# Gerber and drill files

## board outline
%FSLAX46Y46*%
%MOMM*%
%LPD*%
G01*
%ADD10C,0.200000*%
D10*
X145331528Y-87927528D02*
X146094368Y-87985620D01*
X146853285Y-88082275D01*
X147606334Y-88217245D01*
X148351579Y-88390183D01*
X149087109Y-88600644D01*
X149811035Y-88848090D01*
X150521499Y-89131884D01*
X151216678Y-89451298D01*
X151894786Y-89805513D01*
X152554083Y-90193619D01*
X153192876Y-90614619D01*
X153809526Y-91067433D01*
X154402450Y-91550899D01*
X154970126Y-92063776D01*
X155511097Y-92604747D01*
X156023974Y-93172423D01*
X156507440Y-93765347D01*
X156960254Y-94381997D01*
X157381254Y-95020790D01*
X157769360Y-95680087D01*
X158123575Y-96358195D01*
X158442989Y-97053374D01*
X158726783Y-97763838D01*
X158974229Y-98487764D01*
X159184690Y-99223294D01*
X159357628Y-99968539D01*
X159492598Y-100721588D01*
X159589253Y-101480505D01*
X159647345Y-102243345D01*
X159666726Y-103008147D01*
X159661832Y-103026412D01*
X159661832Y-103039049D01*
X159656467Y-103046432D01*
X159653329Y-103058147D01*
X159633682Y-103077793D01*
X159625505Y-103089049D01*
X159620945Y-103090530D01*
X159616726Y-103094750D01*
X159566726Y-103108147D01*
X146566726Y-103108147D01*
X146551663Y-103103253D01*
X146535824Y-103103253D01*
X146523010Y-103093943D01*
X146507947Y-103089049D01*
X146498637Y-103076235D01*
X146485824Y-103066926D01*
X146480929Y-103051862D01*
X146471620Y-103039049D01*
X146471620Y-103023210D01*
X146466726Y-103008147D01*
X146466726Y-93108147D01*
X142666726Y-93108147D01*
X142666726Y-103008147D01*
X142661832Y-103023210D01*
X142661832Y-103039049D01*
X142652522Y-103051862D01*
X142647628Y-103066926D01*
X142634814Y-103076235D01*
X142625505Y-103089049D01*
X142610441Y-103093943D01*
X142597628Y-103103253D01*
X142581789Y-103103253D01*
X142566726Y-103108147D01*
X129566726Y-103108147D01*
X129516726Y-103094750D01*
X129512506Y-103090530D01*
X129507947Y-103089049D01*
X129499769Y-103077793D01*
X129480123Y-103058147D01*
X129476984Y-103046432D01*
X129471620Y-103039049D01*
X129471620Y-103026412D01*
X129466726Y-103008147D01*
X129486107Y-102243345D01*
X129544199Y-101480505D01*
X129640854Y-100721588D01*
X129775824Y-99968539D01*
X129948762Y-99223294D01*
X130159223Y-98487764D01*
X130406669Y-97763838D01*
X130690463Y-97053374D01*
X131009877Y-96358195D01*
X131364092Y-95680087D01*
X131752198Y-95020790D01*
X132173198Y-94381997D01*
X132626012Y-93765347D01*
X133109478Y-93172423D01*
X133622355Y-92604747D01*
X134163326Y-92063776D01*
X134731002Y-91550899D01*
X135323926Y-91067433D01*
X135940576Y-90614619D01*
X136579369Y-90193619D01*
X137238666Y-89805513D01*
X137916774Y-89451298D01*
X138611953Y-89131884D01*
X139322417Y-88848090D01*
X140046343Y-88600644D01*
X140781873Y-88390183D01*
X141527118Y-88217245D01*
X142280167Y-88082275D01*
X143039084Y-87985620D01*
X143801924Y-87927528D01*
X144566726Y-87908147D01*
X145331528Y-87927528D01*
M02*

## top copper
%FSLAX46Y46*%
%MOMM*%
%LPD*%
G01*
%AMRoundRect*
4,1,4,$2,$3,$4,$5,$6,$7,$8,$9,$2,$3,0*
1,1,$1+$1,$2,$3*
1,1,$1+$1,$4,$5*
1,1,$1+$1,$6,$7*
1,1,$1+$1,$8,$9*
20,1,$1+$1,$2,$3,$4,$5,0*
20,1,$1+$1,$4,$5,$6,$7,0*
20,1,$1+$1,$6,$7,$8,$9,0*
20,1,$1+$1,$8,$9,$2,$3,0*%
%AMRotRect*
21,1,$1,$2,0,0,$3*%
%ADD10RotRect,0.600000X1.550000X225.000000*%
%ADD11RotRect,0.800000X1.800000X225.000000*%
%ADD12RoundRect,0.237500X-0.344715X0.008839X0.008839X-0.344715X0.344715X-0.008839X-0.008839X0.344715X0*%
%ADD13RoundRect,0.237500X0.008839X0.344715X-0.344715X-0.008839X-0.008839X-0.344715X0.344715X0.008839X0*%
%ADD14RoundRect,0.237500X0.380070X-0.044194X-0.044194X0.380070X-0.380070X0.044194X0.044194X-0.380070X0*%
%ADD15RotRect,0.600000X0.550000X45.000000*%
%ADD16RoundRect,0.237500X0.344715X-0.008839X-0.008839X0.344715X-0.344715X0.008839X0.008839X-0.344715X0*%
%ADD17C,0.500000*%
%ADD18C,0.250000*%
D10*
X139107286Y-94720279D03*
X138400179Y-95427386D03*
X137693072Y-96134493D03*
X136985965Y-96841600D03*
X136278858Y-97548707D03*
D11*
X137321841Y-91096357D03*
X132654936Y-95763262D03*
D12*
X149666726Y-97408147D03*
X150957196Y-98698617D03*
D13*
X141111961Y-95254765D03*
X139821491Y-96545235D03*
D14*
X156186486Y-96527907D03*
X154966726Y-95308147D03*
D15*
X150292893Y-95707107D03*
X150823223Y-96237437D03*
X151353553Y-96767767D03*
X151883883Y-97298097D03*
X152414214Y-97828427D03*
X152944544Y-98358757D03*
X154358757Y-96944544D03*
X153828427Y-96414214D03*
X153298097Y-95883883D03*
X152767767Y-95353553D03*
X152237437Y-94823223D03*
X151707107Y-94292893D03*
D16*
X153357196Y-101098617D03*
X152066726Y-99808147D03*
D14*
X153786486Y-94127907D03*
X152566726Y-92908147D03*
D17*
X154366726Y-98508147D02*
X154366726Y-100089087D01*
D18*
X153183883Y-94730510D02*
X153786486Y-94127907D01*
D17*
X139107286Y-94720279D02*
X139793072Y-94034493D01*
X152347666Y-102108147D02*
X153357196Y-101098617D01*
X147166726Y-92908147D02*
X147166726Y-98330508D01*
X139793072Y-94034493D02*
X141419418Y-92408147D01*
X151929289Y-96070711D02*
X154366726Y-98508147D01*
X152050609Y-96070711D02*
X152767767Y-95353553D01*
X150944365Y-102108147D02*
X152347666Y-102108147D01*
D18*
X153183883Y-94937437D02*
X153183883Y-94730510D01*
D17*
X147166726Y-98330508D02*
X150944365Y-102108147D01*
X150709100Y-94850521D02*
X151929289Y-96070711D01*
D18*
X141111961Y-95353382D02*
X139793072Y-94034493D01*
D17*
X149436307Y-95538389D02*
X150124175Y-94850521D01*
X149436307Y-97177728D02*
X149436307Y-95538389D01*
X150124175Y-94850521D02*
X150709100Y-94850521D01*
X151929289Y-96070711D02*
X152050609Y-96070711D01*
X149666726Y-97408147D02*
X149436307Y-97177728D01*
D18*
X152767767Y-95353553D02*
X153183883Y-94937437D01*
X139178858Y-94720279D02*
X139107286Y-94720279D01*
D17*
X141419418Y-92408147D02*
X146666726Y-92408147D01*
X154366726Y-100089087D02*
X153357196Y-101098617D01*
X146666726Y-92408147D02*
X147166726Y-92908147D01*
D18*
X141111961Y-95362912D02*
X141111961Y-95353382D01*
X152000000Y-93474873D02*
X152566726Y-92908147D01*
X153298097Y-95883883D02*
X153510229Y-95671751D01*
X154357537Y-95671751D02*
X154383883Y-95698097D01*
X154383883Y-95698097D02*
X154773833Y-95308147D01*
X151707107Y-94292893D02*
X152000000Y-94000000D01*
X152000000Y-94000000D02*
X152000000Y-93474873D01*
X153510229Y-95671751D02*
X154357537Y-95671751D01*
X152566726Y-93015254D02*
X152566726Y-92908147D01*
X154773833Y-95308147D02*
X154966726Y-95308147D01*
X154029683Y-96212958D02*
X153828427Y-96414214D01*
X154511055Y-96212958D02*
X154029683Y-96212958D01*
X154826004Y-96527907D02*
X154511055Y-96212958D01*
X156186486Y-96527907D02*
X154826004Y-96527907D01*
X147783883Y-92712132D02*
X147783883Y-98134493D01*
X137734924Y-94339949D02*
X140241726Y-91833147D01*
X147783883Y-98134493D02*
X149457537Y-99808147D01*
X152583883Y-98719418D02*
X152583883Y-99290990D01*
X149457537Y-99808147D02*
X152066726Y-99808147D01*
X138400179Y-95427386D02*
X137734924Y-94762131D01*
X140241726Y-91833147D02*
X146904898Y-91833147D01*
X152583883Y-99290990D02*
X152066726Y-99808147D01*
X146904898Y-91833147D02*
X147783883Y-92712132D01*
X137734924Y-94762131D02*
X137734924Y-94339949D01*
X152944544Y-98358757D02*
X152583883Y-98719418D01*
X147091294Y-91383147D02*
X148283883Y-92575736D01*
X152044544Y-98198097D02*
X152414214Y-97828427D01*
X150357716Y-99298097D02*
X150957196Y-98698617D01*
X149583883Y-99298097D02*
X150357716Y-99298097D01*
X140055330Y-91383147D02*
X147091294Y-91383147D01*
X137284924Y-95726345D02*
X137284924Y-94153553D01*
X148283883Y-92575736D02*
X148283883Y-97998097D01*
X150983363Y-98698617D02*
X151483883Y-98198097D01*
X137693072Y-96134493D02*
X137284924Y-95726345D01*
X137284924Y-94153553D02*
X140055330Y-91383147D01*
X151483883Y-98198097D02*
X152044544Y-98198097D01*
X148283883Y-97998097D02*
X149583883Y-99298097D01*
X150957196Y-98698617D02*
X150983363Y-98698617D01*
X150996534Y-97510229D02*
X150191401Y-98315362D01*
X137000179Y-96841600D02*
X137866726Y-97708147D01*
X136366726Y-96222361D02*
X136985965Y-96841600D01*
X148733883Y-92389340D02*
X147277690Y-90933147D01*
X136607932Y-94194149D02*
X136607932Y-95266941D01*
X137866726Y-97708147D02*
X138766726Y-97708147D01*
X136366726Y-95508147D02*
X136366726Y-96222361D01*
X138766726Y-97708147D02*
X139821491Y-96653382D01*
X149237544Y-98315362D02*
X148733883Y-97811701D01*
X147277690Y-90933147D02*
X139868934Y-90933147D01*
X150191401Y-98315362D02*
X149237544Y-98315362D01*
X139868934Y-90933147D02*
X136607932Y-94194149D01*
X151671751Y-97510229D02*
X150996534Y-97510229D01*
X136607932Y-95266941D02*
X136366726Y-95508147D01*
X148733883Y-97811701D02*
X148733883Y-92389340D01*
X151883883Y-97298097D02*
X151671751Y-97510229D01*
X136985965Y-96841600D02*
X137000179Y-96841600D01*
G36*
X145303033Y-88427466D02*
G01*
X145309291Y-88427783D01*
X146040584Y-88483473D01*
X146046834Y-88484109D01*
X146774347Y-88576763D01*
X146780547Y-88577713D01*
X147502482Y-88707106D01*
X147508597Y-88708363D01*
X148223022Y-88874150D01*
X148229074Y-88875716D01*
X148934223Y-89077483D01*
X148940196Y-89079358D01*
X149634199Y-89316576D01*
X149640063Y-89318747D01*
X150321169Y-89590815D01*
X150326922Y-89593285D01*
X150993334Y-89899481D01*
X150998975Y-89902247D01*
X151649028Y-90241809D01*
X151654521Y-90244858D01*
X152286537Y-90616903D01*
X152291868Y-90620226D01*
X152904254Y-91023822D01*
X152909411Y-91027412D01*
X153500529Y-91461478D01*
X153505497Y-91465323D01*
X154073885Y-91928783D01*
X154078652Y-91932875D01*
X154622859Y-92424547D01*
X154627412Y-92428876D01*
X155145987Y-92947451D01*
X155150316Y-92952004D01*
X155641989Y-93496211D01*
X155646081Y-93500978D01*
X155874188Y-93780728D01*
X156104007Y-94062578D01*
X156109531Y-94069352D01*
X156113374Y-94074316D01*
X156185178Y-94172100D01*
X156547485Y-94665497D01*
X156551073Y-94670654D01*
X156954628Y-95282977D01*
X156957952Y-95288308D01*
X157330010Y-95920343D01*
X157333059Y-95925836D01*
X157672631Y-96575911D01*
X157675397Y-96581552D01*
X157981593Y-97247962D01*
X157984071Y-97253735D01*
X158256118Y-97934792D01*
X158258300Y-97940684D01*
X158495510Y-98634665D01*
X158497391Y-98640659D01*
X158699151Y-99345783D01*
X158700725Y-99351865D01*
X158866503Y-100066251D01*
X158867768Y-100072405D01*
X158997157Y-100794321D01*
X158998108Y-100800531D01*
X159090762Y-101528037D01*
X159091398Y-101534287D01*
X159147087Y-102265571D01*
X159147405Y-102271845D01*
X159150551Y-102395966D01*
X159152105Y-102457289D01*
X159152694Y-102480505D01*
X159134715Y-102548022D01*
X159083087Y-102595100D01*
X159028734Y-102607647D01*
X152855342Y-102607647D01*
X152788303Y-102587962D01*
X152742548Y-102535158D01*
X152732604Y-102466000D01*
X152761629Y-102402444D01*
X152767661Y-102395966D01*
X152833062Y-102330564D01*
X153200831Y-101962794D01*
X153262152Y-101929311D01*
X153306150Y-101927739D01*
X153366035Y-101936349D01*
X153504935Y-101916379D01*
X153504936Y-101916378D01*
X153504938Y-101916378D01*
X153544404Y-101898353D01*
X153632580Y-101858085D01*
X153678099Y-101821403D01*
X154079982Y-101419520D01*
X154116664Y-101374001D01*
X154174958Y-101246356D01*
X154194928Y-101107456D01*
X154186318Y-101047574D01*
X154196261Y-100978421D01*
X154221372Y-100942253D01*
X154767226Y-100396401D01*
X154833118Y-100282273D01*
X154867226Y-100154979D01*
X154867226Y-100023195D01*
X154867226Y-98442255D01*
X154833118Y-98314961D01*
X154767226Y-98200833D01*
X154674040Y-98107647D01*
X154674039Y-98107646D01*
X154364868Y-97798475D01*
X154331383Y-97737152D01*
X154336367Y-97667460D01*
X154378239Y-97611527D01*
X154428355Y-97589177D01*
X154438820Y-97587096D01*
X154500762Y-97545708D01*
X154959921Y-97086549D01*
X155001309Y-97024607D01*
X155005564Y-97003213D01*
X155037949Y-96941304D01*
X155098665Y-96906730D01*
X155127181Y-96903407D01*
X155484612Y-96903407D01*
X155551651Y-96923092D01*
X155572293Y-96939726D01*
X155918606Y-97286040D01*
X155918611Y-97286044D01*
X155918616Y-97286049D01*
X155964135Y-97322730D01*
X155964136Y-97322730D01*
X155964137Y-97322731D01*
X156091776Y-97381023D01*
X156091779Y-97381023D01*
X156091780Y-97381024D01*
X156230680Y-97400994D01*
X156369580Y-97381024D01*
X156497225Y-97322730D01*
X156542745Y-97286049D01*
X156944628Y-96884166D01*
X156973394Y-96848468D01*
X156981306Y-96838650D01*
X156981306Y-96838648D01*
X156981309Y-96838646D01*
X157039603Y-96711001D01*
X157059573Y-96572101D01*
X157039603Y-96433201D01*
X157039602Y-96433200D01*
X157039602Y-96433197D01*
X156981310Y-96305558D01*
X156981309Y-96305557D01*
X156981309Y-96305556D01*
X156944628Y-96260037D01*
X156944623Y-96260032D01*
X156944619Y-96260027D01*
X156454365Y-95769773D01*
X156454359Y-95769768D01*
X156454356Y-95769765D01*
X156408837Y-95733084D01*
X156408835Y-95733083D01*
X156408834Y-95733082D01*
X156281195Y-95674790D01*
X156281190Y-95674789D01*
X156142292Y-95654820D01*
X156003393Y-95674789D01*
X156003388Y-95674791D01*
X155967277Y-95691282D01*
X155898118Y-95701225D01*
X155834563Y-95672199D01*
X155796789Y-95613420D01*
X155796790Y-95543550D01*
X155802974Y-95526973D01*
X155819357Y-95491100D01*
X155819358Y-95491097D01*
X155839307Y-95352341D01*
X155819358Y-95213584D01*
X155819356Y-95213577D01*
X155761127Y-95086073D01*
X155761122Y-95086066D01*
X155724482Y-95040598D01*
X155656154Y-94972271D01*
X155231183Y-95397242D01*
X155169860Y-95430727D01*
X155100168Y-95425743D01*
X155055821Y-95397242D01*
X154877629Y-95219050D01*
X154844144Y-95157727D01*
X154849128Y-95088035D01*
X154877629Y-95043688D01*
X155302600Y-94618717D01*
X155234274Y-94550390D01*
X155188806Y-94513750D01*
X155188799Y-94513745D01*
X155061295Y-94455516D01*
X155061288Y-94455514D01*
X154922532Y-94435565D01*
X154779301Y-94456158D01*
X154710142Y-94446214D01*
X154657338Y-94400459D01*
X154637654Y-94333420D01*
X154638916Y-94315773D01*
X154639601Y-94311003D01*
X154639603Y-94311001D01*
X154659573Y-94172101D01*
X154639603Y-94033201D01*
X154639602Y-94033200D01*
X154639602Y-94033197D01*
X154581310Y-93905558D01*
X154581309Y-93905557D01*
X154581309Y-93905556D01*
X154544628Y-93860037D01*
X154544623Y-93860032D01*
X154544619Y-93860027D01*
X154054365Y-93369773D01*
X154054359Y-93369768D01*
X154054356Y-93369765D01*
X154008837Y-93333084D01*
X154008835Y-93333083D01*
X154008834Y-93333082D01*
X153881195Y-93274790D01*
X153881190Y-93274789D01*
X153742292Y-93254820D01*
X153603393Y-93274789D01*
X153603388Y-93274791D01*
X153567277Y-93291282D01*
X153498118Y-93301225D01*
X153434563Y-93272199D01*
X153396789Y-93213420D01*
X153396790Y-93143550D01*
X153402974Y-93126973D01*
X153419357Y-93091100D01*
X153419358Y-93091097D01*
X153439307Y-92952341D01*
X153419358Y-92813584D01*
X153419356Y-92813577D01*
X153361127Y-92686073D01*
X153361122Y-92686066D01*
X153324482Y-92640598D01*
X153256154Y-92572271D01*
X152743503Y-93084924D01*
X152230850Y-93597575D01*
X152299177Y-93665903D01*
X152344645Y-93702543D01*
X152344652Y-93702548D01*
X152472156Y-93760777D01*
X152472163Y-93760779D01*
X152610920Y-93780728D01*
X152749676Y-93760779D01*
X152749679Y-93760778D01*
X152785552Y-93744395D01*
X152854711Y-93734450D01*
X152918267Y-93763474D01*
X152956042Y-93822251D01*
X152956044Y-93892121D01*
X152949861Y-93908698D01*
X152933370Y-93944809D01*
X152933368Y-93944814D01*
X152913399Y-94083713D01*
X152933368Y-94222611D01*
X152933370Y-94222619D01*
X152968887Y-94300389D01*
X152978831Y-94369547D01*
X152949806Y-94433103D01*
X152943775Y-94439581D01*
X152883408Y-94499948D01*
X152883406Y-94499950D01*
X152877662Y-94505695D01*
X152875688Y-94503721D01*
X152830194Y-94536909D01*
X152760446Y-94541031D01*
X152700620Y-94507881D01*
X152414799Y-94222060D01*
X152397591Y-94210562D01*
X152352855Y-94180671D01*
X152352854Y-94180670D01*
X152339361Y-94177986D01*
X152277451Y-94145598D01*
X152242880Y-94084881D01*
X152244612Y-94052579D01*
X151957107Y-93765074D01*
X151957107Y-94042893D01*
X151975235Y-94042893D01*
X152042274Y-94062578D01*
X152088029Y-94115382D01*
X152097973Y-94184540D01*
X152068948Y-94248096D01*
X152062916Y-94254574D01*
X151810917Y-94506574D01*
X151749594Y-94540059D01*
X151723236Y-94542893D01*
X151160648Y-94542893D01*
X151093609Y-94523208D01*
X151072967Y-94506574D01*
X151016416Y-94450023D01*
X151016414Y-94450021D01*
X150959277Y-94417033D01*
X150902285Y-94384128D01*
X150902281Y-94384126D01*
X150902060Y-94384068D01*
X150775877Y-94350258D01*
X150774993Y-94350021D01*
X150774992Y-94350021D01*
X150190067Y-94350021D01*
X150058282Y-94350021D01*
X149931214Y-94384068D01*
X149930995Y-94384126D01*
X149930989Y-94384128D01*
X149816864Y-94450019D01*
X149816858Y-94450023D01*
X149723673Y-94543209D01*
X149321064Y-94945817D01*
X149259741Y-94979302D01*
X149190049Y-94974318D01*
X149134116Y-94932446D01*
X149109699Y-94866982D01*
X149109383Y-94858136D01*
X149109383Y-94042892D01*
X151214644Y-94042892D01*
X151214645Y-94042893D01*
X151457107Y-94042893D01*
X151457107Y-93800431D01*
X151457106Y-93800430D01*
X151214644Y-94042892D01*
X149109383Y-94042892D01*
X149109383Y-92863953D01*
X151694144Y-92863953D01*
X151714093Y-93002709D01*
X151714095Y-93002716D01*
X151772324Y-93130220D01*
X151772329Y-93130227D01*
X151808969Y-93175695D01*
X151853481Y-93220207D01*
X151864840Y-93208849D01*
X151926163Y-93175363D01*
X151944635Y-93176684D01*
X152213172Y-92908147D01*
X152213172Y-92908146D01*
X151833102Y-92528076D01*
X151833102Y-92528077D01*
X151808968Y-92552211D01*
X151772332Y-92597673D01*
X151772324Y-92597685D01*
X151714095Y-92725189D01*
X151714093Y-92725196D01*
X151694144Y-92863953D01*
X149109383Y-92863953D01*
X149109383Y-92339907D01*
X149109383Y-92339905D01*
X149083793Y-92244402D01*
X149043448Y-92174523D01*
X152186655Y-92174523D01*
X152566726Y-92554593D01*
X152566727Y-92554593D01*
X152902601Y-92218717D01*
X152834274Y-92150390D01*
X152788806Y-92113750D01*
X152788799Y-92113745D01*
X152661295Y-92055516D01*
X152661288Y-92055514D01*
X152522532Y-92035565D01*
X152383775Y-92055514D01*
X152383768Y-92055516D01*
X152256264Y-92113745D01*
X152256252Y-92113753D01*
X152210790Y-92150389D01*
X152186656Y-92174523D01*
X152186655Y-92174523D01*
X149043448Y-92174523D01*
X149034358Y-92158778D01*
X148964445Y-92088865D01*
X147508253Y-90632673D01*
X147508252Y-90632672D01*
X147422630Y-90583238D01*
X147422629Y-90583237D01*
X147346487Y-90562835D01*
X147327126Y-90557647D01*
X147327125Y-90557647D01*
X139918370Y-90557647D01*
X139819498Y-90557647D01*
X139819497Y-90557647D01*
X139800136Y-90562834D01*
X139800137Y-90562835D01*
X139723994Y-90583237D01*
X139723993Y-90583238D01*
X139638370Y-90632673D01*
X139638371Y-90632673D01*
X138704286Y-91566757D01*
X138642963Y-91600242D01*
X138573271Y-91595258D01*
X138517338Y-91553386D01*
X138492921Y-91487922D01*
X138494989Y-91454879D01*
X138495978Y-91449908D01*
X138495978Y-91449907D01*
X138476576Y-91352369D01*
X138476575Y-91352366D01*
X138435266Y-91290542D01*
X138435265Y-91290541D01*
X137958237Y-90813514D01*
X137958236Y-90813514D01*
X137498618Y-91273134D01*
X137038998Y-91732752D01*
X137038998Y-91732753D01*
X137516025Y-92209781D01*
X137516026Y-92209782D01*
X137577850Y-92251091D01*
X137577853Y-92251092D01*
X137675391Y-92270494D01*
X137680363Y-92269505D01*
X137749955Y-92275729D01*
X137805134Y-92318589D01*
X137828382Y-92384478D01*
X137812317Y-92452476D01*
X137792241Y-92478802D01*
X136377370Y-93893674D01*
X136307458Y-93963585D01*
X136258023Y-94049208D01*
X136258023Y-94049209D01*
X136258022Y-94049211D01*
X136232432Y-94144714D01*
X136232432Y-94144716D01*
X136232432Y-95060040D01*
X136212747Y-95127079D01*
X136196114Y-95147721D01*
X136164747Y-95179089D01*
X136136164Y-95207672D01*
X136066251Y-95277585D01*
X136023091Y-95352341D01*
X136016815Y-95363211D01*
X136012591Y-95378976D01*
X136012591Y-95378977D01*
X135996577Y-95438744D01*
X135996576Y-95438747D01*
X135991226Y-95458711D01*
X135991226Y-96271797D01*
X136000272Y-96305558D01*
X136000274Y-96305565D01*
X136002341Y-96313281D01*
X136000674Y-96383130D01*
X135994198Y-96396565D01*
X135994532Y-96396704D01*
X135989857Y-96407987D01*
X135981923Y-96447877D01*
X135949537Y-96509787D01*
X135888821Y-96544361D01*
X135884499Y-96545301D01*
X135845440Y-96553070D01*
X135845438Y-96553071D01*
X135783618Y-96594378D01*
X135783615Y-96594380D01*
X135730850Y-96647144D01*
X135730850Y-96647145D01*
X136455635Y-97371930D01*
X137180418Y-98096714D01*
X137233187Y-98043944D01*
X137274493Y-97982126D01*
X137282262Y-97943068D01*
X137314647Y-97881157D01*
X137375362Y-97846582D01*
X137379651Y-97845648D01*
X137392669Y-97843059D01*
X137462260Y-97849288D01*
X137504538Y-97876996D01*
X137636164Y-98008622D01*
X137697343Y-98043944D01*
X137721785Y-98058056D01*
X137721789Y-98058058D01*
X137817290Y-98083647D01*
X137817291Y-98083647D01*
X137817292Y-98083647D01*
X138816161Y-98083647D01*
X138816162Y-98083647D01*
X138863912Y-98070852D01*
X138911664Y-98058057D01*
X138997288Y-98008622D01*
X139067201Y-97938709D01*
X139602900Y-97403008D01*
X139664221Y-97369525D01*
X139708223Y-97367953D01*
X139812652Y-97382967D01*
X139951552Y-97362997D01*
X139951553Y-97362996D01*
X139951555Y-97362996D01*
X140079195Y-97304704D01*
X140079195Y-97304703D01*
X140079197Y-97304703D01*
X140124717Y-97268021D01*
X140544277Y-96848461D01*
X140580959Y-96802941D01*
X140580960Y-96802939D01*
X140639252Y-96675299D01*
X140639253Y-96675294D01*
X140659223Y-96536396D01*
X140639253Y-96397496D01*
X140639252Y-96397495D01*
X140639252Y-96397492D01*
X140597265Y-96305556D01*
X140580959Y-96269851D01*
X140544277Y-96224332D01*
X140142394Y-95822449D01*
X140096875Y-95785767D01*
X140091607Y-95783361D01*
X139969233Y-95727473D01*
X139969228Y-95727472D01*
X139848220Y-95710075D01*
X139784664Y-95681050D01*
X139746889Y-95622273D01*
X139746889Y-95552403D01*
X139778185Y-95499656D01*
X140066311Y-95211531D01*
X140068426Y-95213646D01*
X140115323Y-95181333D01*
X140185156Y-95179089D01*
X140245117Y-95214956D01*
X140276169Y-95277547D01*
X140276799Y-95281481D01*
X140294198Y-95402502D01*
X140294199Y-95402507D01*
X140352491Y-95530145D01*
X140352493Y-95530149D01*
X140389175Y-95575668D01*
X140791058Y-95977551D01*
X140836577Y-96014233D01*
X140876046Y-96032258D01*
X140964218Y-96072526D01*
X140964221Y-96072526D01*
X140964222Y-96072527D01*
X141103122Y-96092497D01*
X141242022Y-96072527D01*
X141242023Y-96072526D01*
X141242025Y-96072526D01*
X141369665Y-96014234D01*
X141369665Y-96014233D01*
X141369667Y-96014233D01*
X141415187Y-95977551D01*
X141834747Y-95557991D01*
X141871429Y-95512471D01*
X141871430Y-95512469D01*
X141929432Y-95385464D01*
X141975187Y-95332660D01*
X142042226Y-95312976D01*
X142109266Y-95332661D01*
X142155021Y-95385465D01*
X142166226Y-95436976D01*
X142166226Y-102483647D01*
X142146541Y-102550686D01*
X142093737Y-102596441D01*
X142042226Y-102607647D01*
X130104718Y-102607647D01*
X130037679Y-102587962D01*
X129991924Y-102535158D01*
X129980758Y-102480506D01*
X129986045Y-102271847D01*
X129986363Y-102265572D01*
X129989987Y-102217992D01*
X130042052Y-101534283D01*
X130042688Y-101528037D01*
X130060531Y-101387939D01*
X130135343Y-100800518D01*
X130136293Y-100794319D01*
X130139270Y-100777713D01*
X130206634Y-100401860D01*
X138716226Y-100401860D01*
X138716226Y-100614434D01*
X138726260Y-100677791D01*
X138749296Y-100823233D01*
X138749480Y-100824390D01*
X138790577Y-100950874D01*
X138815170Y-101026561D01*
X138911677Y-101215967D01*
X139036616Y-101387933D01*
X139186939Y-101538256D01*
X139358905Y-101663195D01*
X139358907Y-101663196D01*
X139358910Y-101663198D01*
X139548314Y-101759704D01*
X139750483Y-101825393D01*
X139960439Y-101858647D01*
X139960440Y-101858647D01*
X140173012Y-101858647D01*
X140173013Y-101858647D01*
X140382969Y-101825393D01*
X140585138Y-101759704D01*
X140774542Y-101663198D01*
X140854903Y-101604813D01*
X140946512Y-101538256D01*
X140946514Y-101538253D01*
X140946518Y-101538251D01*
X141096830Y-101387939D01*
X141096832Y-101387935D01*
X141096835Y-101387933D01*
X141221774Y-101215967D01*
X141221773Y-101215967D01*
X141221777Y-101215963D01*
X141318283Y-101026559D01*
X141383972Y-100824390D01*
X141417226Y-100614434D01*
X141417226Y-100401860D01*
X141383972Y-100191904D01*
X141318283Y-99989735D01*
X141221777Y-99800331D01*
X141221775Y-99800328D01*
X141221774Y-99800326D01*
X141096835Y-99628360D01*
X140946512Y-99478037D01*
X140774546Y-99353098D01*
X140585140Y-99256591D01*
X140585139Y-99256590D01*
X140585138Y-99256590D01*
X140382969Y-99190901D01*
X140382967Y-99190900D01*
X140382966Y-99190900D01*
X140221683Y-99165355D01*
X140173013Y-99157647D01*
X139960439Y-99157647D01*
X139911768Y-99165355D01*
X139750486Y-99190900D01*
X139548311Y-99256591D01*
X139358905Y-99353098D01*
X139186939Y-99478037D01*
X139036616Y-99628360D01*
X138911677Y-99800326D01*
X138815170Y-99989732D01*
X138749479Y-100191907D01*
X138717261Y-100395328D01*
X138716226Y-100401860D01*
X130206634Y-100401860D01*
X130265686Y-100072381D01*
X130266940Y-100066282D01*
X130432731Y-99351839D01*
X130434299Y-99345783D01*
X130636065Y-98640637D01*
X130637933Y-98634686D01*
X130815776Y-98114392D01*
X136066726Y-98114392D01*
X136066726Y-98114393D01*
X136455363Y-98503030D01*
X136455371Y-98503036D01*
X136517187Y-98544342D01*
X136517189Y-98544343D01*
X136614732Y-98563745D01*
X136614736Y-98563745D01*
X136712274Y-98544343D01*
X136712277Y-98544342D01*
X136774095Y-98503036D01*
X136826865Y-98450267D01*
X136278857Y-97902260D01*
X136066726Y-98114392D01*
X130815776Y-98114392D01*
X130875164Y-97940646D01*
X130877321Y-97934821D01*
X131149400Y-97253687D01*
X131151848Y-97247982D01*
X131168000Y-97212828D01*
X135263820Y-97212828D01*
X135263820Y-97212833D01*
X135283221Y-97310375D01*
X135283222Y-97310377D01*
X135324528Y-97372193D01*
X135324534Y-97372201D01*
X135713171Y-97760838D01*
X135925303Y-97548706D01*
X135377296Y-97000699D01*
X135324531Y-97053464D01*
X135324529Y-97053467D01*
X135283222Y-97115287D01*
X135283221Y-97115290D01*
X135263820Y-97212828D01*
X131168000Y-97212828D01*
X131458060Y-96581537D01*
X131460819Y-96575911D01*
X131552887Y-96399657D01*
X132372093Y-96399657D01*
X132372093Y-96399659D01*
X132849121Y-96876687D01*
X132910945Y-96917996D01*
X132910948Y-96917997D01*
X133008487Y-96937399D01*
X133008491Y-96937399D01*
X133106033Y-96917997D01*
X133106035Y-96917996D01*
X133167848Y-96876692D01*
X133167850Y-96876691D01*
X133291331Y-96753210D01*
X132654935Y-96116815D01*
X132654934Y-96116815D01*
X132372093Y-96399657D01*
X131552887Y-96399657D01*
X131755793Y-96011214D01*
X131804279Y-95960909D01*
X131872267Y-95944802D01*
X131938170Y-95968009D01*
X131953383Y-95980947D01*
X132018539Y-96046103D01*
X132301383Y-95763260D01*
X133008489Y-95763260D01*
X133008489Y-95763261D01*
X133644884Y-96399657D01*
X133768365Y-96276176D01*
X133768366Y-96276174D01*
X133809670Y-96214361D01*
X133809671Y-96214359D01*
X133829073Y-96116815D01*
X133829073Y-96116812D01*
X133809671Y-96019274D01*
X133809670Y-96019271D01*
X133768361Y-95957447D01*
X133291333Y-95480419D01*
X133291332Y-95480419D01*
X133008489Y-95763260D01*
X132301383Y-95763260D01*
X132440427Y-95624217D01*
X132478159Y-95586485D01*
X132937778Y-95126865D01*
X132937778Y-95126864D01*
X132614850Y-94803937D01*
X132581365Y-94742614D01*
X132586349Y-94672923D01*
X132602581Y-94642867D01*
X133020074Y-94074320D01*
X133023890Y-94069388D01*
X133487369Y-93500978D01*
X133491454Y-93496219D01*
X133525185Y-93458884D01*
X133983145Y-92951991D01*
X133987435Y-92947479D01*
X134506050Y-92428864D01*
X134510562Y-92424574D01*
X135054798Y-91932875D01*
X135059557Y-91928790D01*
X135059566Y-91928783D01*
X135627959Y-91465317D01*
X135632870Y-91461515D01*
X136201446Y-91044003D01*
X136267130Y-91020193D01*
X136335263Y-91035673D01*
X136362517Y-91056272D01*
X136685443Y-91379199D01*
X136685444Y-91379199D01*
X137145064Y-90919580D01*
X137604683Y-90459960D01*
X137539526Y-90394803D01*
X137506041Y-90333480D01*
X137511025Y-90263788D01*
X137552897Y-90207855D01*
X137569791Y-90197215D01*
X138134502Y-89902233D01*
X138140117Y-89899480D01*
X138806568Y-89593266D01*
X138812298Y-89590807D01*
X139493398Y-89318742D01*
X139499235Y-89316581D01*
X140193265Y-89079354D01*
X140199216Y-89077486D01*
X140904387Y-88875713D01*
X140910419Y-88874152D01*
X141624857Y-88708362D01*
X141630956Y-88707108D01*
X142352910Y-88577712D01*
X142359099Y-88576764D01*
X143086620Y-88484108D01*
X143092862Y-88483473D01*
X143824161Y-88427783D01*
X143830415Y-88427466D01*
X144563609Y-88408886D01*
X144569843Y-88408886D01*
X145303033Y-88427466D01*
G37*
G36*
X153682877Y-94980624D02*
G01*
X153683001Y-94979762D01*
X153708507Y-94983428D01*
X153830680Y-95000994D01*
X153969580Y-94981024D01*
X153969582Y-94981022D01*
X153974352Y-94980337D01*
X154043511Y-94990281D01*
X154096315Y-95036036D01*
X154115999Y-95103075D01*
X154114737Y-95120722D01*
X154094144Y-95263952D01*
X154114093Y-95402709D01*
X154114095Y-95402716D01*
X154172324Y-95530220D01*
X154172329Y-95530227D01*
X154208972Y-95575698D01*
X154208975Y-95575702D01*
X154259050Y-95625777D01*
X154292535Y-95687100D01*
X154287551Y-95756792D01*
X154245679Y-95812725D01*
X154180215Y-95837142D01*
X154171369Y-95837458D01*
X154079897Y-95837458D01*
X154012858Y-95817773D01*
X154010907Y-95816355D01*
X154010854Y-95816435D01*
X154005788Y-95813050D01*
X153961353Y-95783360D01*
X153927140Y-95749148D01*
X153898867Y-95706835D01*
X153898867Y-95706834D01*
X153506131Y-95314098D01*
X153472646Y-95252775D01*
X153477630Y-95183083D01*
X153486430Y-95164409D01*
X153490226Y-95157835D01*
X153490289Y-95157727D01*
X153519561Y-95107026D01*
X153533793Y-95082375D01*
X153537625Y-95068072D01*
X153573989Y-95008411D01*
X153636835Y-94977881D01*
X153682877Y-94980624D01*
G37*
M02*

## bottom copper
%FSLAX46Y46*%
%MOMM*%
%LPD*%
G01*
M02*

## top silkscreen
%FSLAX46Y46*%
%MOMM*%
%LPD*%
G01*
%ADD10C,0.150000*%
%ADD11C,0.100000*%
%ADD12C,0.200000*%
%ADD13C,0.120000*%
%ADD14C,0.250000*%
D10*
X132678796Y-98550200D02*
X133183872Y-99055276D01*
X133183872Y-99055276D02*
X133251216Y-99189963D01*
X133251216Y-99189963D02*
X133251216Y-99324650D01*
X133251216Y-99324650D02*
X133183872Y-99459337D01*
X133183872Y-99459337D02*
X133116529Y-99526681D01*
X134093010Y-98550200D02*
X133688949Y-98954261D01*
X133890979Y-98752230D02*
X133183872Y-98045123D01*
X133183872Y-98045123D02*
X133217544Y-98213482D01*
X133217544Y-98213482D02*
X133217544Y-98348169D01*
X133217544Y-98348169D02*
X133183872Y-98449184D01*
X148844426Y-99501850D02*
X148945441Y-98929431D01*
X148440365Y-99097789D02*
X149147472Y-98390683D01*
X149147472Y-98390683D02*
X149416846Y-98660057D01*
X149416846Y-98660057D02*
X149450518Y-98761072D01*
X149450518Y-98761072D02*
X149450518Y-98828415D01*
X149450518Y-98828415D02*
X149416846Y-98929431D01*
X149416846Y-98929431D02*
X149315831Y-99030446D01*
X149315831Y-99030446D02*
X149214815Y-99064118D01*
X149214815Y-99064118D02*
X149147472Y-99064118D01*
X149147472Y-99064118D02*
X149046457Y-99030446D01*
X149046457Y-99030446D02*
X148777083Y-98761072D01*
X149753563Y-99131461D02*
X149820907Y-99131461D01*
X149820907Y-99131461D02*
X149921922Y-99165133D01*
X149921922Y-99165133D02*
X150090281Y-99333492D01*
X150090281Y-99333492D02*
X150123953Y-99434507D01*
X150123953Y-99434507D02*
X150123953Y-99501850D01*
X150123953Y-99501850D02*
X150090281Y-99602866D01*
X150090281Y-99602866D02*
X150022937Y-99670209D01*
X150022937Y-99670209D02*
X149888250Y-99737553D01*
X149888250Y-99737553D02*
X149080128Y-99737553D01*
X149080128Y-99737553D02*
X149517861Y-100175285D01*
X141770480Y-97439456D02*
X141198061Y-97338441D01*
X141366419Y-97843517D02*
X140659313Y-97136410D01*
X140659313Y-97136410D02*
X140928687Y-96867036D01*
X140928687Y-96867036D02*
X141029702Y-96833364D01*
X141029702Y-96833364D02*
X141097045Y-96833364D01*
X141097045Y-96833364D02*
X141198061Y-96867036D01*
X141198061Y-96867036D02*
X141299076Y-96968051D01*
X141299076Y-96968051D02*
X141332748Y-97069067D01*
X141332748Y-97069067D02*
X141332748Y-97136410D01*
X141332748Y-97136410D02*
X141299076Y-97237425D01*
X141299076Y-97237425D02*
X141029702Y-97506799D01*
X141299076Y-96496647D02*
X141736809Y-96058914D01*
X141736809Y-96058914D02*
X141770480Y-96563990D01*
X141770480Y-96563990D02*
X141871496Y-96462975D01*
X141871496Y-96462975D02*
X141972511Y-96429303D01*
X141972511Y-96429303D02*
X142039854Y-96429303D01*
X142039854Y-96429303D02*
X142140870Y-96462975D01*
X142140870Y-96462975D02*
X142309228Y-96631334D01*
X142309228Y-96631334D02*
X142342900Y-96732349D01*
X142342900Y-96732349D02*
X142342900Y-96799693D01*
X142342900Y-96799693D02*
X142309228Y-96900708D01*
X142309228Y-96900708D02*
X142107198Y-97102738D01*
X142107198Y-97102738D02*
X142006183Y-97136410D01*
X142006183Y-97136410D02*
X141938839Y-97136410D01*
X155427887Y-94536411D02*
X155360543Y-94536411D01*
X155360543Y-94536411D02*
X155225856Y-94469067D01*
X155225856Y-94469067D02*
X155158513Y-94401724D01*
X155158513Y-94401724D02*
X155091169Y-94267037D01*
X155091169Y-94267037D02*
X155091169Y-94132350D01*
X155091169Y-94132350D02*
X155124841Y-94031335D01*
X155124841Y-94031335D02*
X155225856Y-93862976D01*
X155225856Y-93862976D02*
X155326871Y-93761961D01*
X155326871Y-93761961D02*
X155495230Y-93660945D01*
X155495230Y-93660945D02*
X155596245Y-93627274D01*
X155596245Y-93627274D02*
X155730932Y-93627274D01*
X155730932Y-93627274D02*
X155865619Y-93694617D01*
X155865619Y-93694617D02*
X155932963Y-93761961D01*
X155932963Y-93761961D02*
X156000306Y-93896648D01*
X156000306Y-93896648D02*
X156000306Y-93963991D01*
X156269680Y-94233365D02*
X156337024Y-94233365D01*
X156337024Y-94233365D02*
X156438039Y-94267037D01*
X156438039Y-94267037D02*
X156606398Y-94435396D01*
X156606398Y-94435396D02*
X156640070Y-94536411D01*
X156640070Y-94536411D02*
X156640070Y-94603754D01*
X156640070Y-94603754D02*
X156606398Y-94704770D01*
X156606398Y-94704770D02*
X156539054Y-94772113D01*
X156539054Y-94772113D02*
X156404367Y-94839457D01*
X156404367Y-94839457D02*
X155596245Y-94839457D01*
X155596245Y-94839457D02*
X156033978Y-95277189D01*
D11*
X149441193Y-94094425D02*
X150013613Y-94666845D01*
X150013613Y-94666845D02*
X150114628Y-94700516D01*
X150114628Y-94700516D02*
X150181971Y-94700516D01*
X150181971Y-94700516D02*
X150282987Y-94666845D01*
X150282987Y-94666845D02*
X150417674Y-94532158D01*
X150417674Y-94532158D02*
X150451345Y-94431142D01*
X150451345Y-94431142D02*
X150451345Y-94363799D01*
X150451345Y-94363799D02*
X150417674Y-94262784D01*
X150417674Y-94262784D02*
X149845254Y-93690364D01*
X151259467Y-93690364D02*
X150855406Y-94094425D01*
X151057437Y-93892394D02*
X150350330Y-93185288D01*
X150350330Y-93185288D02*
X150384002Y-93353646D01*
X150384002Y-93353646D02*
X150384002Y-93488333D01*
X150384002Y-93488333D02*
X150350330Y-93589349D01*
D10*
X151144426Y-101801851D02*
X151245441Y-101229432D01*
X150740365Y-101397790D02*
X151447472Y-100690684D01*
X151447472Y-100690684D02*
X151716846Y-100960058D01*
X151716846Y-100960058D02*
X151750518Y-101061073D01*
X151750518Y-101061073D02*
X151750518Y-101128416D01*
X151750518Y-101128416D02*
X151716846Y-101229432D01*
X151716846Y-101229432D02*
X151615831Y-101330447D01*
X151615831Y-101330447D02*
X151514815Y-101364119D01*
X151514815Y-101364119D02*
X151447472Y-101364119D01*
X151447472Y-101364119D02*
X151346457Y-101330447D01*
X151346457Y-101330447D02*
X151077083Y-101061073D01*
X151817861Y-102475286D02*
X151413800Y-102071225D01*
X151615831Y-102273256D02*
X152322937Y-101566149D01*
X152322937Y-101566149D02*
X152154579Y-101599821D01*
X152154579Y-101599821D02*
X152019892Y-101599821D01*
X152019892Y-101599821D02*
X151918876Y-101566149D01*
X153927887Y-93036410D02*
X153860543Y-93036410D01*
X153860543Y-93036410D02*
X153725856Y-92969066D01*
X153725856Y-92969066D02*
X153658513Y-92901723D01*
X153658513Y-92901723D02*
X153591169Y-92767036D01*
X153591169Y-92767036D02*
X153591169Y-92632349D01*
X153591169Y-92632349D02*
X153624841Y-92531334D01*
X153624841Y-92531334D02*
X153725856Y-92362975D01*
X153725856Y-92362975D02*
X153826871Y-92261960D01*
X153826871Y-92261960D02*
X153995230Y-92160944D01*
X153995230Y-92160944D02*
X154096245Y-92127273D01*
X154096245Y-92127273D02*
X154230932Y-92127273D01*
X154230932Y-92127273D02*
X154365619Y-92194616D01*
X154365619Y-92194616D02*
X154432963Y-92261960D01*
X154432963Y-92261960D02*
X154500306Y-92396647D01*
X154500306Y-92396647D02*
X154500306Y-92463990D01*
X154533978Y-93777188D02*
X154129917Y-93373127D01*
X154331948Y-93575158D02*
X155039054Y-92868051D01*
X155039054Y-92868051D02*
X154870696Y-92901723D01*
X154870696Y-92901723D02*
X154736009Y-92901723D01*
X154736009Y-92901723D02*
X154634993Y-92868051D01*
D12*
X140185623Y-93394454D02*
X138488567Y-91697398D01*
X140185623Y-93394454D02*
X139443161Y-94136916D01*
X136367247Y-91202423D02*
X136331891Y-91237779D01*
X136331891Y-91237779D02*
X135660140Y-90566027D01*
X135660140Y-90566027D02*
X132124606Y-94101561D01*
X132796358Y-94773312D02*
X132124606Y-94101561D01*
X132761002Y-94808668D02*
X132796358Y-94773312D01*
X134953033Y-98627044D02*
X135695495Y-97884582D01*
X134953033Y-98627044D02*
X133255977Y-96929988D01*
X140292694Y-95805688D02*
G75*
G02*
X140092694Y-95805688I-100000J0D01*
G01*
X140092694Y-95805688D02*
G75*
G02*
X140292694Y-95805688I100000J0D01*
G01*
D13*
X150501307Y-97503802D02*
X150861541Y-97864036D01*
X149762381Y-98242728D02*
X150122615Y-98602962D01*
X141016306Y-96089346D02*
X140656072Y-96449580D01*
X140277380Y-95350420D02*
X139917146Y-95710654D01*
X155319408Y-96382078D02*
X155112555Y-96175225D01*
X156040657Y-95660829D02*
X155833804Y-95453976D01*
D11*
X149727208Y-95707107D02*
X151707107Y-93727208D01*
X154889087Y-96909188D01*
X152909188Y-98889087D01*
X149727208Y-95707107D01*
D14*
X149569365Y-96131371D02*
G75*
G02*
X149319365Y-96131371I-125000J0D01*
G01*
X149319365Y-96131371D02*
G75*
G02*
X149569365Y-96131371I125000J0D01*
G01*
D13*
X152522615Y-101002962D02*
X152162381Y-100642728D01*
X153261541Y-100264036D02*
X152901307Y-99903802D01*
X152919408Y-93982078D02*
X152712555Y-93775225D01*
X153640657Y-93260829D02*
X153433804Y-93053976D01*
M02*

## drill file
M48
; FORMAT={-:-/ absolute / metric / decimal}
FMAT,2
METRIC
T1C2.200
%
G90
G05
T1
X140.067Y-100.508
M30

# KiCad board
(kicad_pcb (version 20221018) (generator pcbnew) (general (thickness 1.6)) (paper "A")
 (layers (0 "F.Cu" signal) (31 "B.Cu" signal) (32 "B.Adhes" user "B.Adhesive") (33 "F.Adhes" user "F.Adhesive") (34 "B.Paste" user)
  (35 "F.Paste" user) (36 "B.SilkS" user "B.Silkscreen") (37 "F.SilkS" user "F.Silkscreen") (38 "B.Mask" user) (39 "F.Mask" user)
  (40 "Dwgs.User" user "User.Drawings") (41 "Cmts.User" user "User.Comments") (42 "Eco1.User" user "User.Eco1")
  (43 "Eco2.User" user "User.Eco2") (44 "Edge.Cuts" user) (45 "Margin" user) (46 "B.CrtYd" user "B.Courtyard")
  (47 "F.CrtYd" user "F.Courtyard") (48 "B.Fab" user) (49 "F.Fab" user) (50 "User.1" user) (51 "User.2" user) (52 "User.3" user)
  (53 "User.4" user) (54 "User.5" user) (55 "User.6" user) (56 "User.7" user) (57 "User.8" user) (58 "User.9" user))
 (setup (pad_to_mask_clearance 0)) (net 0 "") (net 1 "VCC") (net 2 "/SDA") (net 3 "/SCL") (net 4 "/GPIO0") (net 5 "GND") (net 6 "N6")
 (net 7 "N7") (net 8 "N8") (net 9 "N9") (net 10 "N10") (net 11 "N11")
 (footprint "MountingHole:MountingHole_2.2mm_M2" (layer "F.Cu") (at 140.066726 100.508147)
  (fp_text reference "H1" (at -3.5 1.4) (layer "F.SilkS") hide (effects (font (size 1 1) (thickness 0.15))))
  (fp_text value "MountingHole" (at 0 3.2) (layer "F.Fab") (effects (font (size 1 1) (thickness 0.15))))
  (pad "" np_thru_hole circle (at 0 0) (size 2.2 2.2) (drill 2.2) (layers "*.Cu" "*.Mask")))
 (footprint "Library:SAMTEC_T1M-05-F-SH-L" (layer "F.Cu") (at 137.693072 96.134493 -135)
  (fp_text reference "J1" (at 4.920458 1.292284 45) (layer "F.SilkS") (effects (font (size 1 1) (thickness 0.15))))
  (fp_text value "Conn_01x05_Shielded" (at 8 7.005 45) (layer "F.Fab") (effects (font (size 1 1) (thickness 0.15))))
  (fp_line (start -3.7 0.175) (end -3.7 2.575) (stroke (width 0.2) (type solid)) (layer "F.SilkS"))
  (fp_line (start -3.7 0.175) (end -2.65 0.175) (stroke (width 0.2) (type solid)) (layer "F.SilkS"))
  (fp_line (start -2.55 4.425) (end -2.5 4.425) (stroke (width 0.2) (type solid)) (layer "F.SilkS"))
  (fp_line (start -2.5 4.425) (end -2.5 5.375) (stroke (width 0.2) (type solid)) (layer "F.SilkS"))
  (fp_line (start -2.5 5.375) (end 2.5 5.375) (stroke (width 0.2) (type solid)) (layer "F.SilkS"))
  (fp_line (start 2.5 4.425) (end 2.5 5.375) (stroke (width 0.2) (type solid)) (layer "F.SilkS"))
  (fp_line (start 2.55 4.425) (end 2.5 4.425) (stroke (width 0.2) (type solid)) (layer "F.SilkS"))
  (fp_line (start 3.7 0.175) (end 2.65 0.175) (stroke (width 0.2) (type solid)) (layer "F.SilkS"))
  (fp_line (start 3.7 0.175) (end 3.7 2.575) (stroke (width 0.2) (type solid)) (layer "F.SilkS"))
  (fp_circle (center -2 -1.535) (end -1.9 -1.535) (stroke (width 0.2) (type solid)) (fill none) (layer "F.SilkS"))
  (pad "1" smd rect (at -2 0 225) (size 0.6 1.55) (layers "F.Cu" "F.Paste" "F.Mask") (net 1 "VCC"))
  (pad "2" smd rect (at -1 0 225) (size 0.6 1.55) (layers "F.Cu" "F.Paste" "F.Mask") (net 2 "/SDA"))
  (pad "3" smd rect (at 0 0 225) (size 0.6 1.55) (layers "F.Cu" "F.Paste" "F.Mask") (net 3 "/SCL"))
  (pad "4" smd rect (at 1 0 225) (size 0.6 1.55) (layers "F.Cu" "F.Paste" "F.Mask") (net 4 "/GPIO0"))
  (pad "5" smd rect (at 2 0 225) (size 0.6 1.55) (layers "F.Cu" "F.Paste" "F.Mask") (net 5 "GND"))
  (pad "SH1" smd rect (at -3.3 3.825 225) (size 0.8 1.8) (layers "F.Cu" "F.Paste" "F.Mask") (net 5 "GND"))
  (pad "SH2" smd rect (at 3.3 3.825 225) (size 0.8 1.8) (layers "F.Cu" "F.Paste" "F.Mask") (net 5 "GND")))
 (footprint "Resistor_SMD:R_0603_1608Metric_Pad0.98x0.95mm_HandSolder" (layer "F.Cu") (at 150.311961 98.053382 -45)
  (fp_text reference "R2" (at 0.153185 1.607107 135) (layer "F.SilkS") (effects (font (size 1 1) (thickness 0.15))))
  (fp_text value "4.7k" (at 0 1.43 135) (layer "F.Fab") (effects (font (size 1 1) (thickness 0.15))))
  (fp_line (start -0.254724 -0.5225) (end 0.254724 -0.5225) (stroke (width 0.12) (type solid)) (layer "F.SilkS"))
  (fp_line (start -0.254724 0.5225) (end 0.254724 0.5225) (stroke (width 0.12) (type solid)) (layer "F.SilkS"))
  (pad "1" smd roundrect (at -0.9125 0 315) (size 0.975 0.95) (layers "F.Cu" "F.Paste" "F.Mask") (roundrect_rratio 0.25) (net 1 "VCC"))
  (pad "2" smd roundrect (at 0.9125 0 315) (size 0.975 0.95) (layers "F.Cu" "F.Paste" "F.Mask") (roundrect_rratio 0.25) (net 3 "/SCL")))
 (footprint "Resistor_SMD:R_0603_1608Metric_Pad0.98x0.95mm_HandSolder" (layer "F.Cu") (at 140.466726 95.9 -135)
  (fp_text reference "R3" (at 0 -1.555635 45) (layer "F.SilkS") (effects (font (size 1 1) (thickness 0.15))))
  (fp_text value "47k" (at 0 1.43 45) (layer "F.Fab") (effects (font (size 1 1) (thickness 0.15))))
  (fp_line (start -0.254724 -0.5225) (end 0.254724 -0.5225) (stroke (width 0.12) (type solid)) (layer "F.SilkS"))
  (fp_line (start -0.254724 0.5225) (end 0.254724 0.5225) (stroke (width 0.12) (type solid)) (layer "F.SilkS"))
  (pad "1" smd roundrect (at -0.9125 0 225) (size 0.975 0.95) (layers "F.Cu" "F.Paste" "F.Mask") (roundrect_rratio 0.25) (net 1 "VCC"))
  (pad "2" smd roundrect (at 0.9125 0 225) (size 0.975 0.95) (layers "F.Cu" "F.Paste" "F.Mask") (roundrect_rratio 0.25) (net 4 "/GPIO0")))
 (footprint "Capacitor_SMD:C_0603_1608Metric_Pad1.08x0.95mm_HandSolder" (layer "F.Cu") (at 155.576606 95.918027 135)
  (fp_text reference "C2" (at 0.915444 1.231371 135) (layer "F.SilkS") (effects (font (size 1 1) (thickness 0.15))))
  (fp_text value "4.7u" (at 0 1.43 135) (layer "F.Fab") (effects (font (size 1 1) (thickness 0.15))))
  (fp_line (start -0.146267 -0.51) (end 0.146267 -0.51) (stroke (width 0.12) (type solid)) (layer "F.SilkS"))
  (fp_line (start -0.146267 0.51) (end 0.146267 0.51) (stroke (width 0.12) (type solid)) (layer "F.SilkS"))
  (pad "1" smd roundrect (at -0.8625 0 135) (size 1.075 0.95) (layers "F.Cu" "F.Paste" "F.Mask") (roundrect_rratio 0.25) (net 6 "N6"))
  (pad "2" smd roundrect (at 0.8625 0 135) (size 1.075 0.95) (layers "F.Cu" "F.Paste" "F.Mask") (roundrect_rratio 0.25) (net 5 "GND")))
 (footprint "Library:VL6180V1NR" (layer "F.Cu") (at 151 95 45)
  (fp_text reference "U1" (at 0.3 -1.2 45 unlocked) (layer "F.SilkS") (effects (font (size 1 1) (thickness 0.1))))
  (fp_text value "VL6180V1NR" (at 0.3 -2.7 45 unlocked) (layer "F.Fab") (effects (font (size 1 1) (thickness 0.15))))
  (fp_rect (start -1.4 -0.4) (end 1.4 4.1) (stroke (width 0.1) (type default)) (fill none) (layer "F.SilkS"))
  (fp_circle (center -1.9 -0.3) (end -1.7 -0.3) (stroke (width 0.1) (type solid)) (fill solid) (layer "F.SilkS"))
  (pad "1" smd rect (at -1 0 45) (size 0.6 0.55) (layers "F.Cu" "F.Paste" "F.Mask") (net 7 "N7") (thermal_bridge_angle 45))
  (pad "2" smd rect (at -1 0.75 45) (size 0.6 0.55) (layers "F.Cu" "F.Paste" "F.Mask") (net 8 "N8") (thermal_bridge_angle 45))
  (pad "3" smd rect (at -1 1.5 45) (size 0.6 0.55) (layers "F.Cu" "F.Paste" "F.Mask") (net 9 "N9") (thermal_bridge_angle 45))
  (pad "4" smd rect (at -1 2.25 45) (size 0.6 0.55) (layers "F.Cu" "F.Paste" "F.Mask") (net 4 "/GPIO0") (thermal_bridge_angle 45))
  (pad "5" smd rect (at -1 3 45) (size 0.6 0.55) (layers "F.Cu" "F.Paste" "F.Mask") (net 3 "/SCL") (thermal_bridge_angle 45))
  (pad "6" smd rect (at -1 3.75 45) (size 0.6 0.55) (layers "F.Cu" "F.Paste" "F.Mask") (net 2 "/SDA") (thermal_bridge_angle 45))
  (pad "7" smd rect (at 1 3.75 45) (size 0.6 0.55) (layers "F.Cu" "F.Paste" "F.Mask") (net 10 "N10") (thermal_bridge_angle 45))
  (pad "8" smd rect (at 1 3 45) (size 0.6 0.55) (layers "F.Cu" "F.Paste" "F.Mask") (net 6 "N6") (thermal_bridge_angle 45))
  (pad "9" smd rect (at 1 2.25 45) (size 0.6 0.55) (layers "F.Cu" "F.Paste" "F.Mask") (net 5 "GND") (thermal_bridge_angle 45))
  (pad "10" smd rect (at 1 1.5 45) (size 0.6 0.55) (layers "F.Cu" "F.Paste" "F.Mask") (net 1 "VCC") (thermal_bridge_angle 45))
  (pad "11" smd rect (at 1 0.75 45) (size 0.6 0.55) (layers "F.Cu" "F.Paste" "F.Mask") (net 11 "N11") (thermal_bridge_angle 45))
  (pad "12" smd rect (at 1 0 45) (size 0.6 0.55) (layers "F.Cu" "F.Paste" "F.Mask") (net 5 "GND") (thermal_bridge_angle 45)))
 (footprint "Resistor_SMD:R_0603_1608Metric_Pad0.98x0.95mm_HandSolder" (layer "F.Cu") (at 152.711961 100.453382 135)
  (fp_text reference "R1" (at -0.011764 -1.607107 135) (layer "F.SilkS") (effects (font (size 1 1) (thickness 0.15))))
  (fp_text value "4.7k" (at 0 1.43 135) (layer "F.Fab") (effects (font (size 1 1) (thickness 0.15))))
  (fp_line (start -0.254724 -0.5225) (end 0.254724 -0.5225) (stroke (width 0.12) (type solid)) (layer "F.SilkS"))
  (fp_line (start -0.254724 0.5225) (end 0.254724 0.5225) (stroke (width 0.12) (type solid)) (layer "F.SilkS"))
  (pad "1" smd roundrect (at -0.9125 0 135) (size 0.975 0.95) (layers "F.Cu" "F.Paste" "F.Mask") (roundrect_rratio 0.25) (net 1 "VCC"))
  (pad "2" smd roundrect (at 0.9125 0 135) (size 0.975 0.95) (layers "F.Cu" "F.Paste" "F.Mask") (roundrect_rratio 0.25) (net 2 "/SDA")))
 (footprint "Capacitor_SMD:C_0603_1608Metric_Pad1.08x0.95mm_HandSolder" (layer "F.Cu") (at 153.176606 93.518027 135)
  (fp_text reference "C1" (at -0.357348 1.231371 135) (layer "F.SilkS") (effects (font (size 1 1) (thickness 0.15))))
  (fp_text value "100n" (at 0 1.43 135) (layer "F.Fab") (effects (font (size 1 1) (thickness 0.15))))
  (fp_line (start -0.146267 -0.51) (end 0.146267 -0.51) (stroke (width 0.12) (type solid)) (layer "F.SilkS"))
  (fp_line (start -0.146267 0.51) (end 0.146267 0.51) (stroke (width 0.12) (type solid)) (layer "F.SilkS"))
  (pad "1" smd roundrect (at -0.8625 0 135) (size 1.075 0.95) (layers "F.Cu" "F.Paste" "F.Mask") (roundrect_rratio 0.25) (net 1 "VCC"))
  (pad "2" smd roundrect (at 0.8625 0 135) (size 1.075 0.95) (layers "F.Cu" "F.Paste" "F.Mask") (roundrect_rratio 0.25) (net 5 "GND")))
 (gr_poly
  (pts (xy 145.331528 87.927528) (xy 146.094368 87.98562) (xy 146.853285 88.082275) (xy 147.606334 88.217245) (xy 148.351579 88.390183)
   (xy 149.087109 88.600644) (xy 149.811035 88.84809) (xy 150.521499 89.131884) (xy 151.216678 89.451298) (xy 151.894786 89.805513)
   (xy 152.554083 90.193619) (xy 153.192876 90.614619) (xy 153.809526 91.067433) (xy 154.40245 91.550899) (xy 154.970126 92.063776)
   (xy 155.511097 92.604747) (xy 156.023974 93.172423) (xy 156.50744 93.765347) (xy 156.960254 94.381997) (xy 157.381254 95.02079)
   (xy 157.76936 95.680087) (xy 158.123575 96.358195) (xy 158.442989 97.053374) (xy 158.726783 97.763838) (xy 158.974229 98.487764)
   (xy 159.18469 99.223294) (xy 159.357628 99.968539) (xy 159.492598 100.721588) (xy 159.589253 101.480505) (xy 159.647345 102.243345)
   (xy 159.666726 103.008147) (xy 159.661832 103.026412) (xy 159.661832 103.039049) (xy 159.656467 103.046432) (xy 159.653329 103.058147)
   (xy 159.633682 103.077793) (xy 159.625505 103.089049) (xy 159.620945 103.09053) (xy 159.616726 103.09475) (xy 159.566726 103.108147)
   (xy 146.566726 103.108147) (xy 146.551663 103.103253) (xy 146.535824 103.103253) (xy 146.52301 103.093943) (xy 146.507947 103.089049)
   (xy 146.498637 103.076235) (xy 146.485824 103.066926) (xy 146.480929 103.051862) (xy 146.47162 103.039049) (xy 146.47162 103.02321)
   (xy 146.466726 103.008147) (xy 146.466726 93.108147) (xy 142.666726 93.108147) (xy 142.666726 103.008147) (xy 142.661832 103.02321)
   (xy 142.661832 103.039049) (xy 142.652522 103.051862) (xy 142.647628 103.066926) (xy 142.634814 103.076235) (xy 142.625505 103.089049)
   (xy 142.610441 103.093943) (xy 142.597628 103.103253) (xy 142.581789 103.103253) (xy 142.566726 103.108147) (xy 129.566726 103.108147)
   (xy 129.516726 103.09475) (xy 129.512506 103.09053) (xy 129.507947 103.089049) (xy 129.499769 103.077793) (xy 129.480123 103.058147)
   (xy 129.476984 103.046432) (xy 129.47162 103.039049) (xy 129.47162 103.026412) (xy 129.466726 103.008147) (xy 129.486107 102.243345)
   (xy 129.544199 101.480505) (xy 129.640854 100.721588) (xy 129.775824 99.968539) (xy 129.948762 99.223294) (xy 130.159223 98.487764)
   (xy 130.406669 97.763838) (xy 130.690463 97.053374) (xy 131.009877 96.358195) (xy 131.364092 95.680087) (xy 131.752198 95.02079)
   (xy 132.173198 94.381997) (xy 132.626012 93.765347) (xy 133.109478 93.172423) (xy 133.622355 92.604747) (xy 134.163326 92.063776)
   (xy 134.731002 91.550899) (xy 135.323926 91.067433) (xy 135.940576 90.614619) (xy 136.579369 90.193619) (xy 137.238666 89.805513)
   (xy 137.916774 89.451298) (xy 138.611953 89.131884) (xy 139.322417 88.84809) (xy 140.046343 88.600644) (xy 140.781873 88.390183)
   (xy 141.527118 88.217245) (xy 142.280167 88.082275) (xy 143.039084 87.98562) (xy 143.801924 87.927528) (xy 144.566726 87.908147))
  (stroke (width 0.2) (type solid)) (fill none) (layer "Edge.Cuts"))
 (segment (start 154.366726 98.508147) (end 154.366726 100.089087) (width 0.5) (layer "F.Cu") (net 1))
 (segment (start 153.183883 94.73051) (end 153.786486 94.127907) (width 0.25) (layer "F.Cu") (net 1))
 (segment (start 139.107286 94.720279) (end 139.793072 94.034493) (width 0.5) (layer "F.Cu") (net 1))
 (segment (start 152.347666 102.108147) (end 153.357196 101.098617) (width 0.5) (layer "F.Cu") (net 1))
 (segment (start 147.166726 92.908147) (end 147.166726 98.330508) (width 0.5) (layer "F.Cu") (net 1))
 (segment (start 139.793072 94.034493) (end 141.419418 92.408147) (width 0.5) (layer "F.Cu") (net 1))
 (segment (start 151.929289 96.070711) (end 154.366726 98.508147) (width 0.5) (layer "F.Cu") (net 1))
 (segment (start 152.050609 96.070711) (end 152.767767 95.353553) (width 0.5) (layer "F.Cu") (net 1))
 (segment (start 150.944365 102.108147) (end 152.347666 102.108147) (width 0.5) (layer "F.Cu") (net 1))
 (segment (start 153.183883 94.937437) (end 153.183883 94.73051) (width 0.25) (layer "F.Cu") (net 1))
 (segment (start 147.166726 98.330508) (end 150.944365 102.108147) (width 0.5) (layer "F.Cu") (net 1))
 (segment (start 150.7091 94.850521) (end 151.929289 96.070711) (width 0.5) (layer "F.Cu") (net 1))
 (segment (start 141.111961 95.353382) (end 139.793072 94.034493) (width 0.25) (layer "F.Cu") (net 1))
 (segment (start 149.436307 95.538389) (end 150.124175 94.850521) (width 0.5) (layer "F.Cu") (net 1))
 (segment (start 149.436307 97.177728) (end 149.436307 95.538389) (width 0.5) (layer "F.Cu") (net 1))
 (segment (start 150.124175 94.850521) (end 150.7091 94.850521) (width 0.5) (layer "F.Cu") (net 1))
 (segment (start 151.929289 96.070711) (end 152.050609 96.070711) (width 0.5) (layer "F.Cu") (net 1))
 (segment (start 149.666726 97.408147) (end 149.436307 97.177728) (width 0.5) (layer "F.Cu") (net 1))
 (segment (start 152.767767 95.353553) (end 153.183883 94.937437) (width 0.25) (layer "F.Cu") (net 1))
 (segment (start 139.178858 94.720279) (end 139.107286 94.720279) (width 0.25) (layer "F.Cu") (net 1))
 (segment (start 141.419418 92.408147) (end 146.666726 92.408147) (width 0.5) (layer "F.Cu") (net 1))
 (segment (start 154.366726 100.089087) (end 153.357196 101.098617) (width 0.5) (layer "F.Cu") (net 1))
 (segment (start 146.666726 92.408147) (end 147.166726 92.908147) (width 0.5) (layer "F.Cu") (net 1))
 (segment (start 141.111961 95.362912) (end 141.111961 95.353382) (width 0.25) (layer "F.Cu") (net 1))
 (segment (start 152 93.474873) (end 152.566726 92.908147) (width 0.25) (layer "F.Cu") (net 5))
 (segment (start 153.298097 95.883883) (end 153.510229 95.671751) (width 0.25) (layer "F.Cu") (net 5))
 (segment (start 154.357537 95.671751) (end 154.383883 95.698097) (width 0.25) (layer "F.Cu") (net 5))
 (segment (start 154.383883 95.698097) (end 154.773833 95.308147) (width 0.25) (layer "F.Cu") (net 5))
 (segment (start 151.707107 94.292893) (end 152 94) (width 0.25) (layer "F.Cu") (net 5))
 (segment (start 152 94) (end 152 93.474873) (width 0.25) (layer "F.Cu") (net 5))
 (segment (start 153.510229 95.671751) (end 154.357537 95.671751) (width 0.25) (layer "F.Cu") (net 5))
 (segment (start 152.566726 93.015254) (end 152.566726 92.908147) (width 0.25) (layer "F.Cu") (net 5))
 (segment (start 154.773833 95.308147) (end 154.966726 95.308147) (width 0.25) (layer "F.Cu") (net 5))
 (segment (start 154.029683 96.212958) (end 153.828427 96.414214) (width 0.25) (layer "F.Cu") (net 6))
 (segment (start 154.511055 96.212958) (end 154.029683 96.212958) (width 0.25) (layer "F.Cu") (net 6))
 (segment (start 154.826004 96.527907) (end 154.511055 96.212958) (width 0.25) (layer "F.Cu") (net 6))
 (segment (start 156.186486 96.527907) (end 154.826004 96.527907) (width 0.25) (layer "F.Cu") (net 6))
 (segment (start 147.783883 92.712132) (end 147.783883 98.134493) (width 0.25) (layer "F.Cu") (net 2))
 (segment (start 137.734924 94.339949) (end 140.241726 91.833147) (width 0.25) (layer "F.Cu") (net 2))
 (segment (start 147.783883 98.134493) (end 149.457537 99.808147) (width 0.25) (layer "F.Cu") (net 2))
 (segment (start 152.583883 98.719418) (end 152.583883 99.29099) (width 0.25) (layer "F.Cu") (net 2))
 (segment (start 149.457537 99.808147) (end 152.066726 99.808147) (width 0.25) (layer "F.Cu") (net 2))
 (segment (start 138.400179 95.427386) (end 137.734924 94.762131) (width 0.25) (layer "F.Cu") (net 2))
 (segment (start 140.241726 91.833147) (end 146.904898 91.833147) (width 0.25) (layer "F.Cu") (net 2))
 (segment (start 152.583883 99.29099) (end 152.066726 99.808147) (width 0.25) (layer "F.Cu") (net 2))
 (segment (start 146.904898 91.833147) (end 147.783883 92.712132) (width 0.25) (layer "F.Cu") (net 2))
 (segment (start 137.734924 94.762131) (end 137.734924 94.339949) (width 0.25) (layer "F.Cu") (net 2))
 (segment (start 152.944544 98.358757) (end 152.583883 98.719418) (width 0.25) (layer "F.Cu") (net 2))
 (segment (start 147.091294 91.383147) (end 148.283883 92.575736) (width 0.25) (layer "F.Cu") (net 3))
 (segment (start 152.044544 98.198097) (end 152.414214 97.828427) (width 0.25) (layer "F.Cu") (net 3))
 (segment (start 150.357716 99.298097) (end 150.957196 98.698617) (width 0.25) (layer "F.Cu") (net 3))
 (segment (start 149.583883 99.298097) (end 150.357716 99.298097) (width 0.25) (layer "F.Cu") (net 3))
 (segment (start 140.05533 91.383147) (end 147.091294 91.383147) (width 0.25) (layer "F.Cu") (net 3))
 (segment (start 137.284924 95.726345) (end 137.284924 94.153553) (width 0.25) (layer "F.Cu") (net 3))
 (segment (start 148.283883 92.575736) (end 148.283883 97.998097) (width 0.25) (layer "F.Cu") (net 3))
 (segment (start 150.983363 98.698617) (end 151.483883 98.198097) (width 0.25) (layer "F.Cu") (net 3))
 (segment (start 137.693072 96.134493) (end 137.284924 95.726345) (width 0.25) (layer "F.Cu") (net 3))
 (segment (start 137.284924 94.153553) (end 140.05533 91.383147) (width 0.25) (layer "F.Cu") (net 3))
 (segment (start 151.483883 98.198097) (end 152.044544 98.198097) (width 0.25) (layer "F.Cu") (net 3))
 (segment (start 148.283883 97.998097) (end 149.583883 99.298097) (width 0.25) (layer "F.Cu") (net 3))
 (segment (start 150.957196 98.698617) (end 150.983363 98.698617) (width 0.25) (layer "F.Cu") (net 3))
 (segment (start 150.996534 97.510229) (end 150.191401 98.315362) (width 0.25) (layer "F.Cu") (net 4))
 (segment (start 137.000179 96.8416) (end 137.866726 97.708147) (width 0.25) (layer "F.Cu") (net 4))
 (segment (start 136.366726 96.222361) (end 136.985965 96.8416) (width 0.25) (layer "F.Cu") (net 4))
 (segment (start 148.733883 92.38934) (end 147.27769 90.933147) (width 0.25) (layer "F.Cu") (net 4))
 (segment (start 136.607932 94.194149) (end 136.607932 95.266941) (width 0.25) (layer "F.Cu") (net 4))
 (segment (start 137.866726 97.708147) (end 138.766726 97.708147) (width 0.25) (layer "F.Cu") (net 4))
 (segment (start 136.366726 95.508147) (end 136.366726 96.222361) (width 0.25) (layer "F.Cu") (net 4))
 (segment (start 138.766726 97.708147) (end 139.821491 96.653382) (width 0.25) (layer "F.Cu") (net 4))
 (segment (start 149.237544 98.315362) (end 148.733883 97.811701) (width 0.25) (layer "F.Cu") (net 4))
 (segment (start 147.27769 90.933147) (end 139.868934 90.933147) (width 0.25) (layer "F.Cu") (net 4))
 (segment (start 150.191401 98.315362) (end 149.237544 98.315362) (width 0.25) (layer "F.Cu") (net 4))
 (segment (start 139.868934 90.933147) (end 136.607932 94.194149) (width 0.25) (layer "F.Cu") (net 4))
 (segment (start 151.671751 97.510229) (end 150.996534 97.510229) (width 0.25) (layer "F.Cu") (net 4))
 (segment (start 136.607932 95.266941) (end 136.366726 95.508147) (width 0.25) (layer "F.Cu") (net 4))
 (segment (start 148.733883 97.811701) (end 148.733883 92.38934) (width 0.25) (layer "F.Cu") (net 4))
 (segment (start 151.883883 97.298097) (end 151.671751 97.510229) (width 0.25) (layer "F.Cu") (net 4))
 (segment (start 136.985965 96.8416) (end 137.000179 96.8416) (width 0.25) (layer "F.Cu") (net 4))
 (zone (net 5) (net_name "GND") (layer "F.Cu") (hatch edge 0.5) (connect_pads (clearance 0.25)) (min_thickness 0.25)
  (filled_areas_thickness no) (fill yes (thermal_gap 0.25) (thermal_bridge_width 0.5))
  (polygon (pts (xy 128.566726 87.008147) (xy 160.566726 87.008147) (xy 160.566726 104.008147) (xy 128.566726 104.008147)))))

